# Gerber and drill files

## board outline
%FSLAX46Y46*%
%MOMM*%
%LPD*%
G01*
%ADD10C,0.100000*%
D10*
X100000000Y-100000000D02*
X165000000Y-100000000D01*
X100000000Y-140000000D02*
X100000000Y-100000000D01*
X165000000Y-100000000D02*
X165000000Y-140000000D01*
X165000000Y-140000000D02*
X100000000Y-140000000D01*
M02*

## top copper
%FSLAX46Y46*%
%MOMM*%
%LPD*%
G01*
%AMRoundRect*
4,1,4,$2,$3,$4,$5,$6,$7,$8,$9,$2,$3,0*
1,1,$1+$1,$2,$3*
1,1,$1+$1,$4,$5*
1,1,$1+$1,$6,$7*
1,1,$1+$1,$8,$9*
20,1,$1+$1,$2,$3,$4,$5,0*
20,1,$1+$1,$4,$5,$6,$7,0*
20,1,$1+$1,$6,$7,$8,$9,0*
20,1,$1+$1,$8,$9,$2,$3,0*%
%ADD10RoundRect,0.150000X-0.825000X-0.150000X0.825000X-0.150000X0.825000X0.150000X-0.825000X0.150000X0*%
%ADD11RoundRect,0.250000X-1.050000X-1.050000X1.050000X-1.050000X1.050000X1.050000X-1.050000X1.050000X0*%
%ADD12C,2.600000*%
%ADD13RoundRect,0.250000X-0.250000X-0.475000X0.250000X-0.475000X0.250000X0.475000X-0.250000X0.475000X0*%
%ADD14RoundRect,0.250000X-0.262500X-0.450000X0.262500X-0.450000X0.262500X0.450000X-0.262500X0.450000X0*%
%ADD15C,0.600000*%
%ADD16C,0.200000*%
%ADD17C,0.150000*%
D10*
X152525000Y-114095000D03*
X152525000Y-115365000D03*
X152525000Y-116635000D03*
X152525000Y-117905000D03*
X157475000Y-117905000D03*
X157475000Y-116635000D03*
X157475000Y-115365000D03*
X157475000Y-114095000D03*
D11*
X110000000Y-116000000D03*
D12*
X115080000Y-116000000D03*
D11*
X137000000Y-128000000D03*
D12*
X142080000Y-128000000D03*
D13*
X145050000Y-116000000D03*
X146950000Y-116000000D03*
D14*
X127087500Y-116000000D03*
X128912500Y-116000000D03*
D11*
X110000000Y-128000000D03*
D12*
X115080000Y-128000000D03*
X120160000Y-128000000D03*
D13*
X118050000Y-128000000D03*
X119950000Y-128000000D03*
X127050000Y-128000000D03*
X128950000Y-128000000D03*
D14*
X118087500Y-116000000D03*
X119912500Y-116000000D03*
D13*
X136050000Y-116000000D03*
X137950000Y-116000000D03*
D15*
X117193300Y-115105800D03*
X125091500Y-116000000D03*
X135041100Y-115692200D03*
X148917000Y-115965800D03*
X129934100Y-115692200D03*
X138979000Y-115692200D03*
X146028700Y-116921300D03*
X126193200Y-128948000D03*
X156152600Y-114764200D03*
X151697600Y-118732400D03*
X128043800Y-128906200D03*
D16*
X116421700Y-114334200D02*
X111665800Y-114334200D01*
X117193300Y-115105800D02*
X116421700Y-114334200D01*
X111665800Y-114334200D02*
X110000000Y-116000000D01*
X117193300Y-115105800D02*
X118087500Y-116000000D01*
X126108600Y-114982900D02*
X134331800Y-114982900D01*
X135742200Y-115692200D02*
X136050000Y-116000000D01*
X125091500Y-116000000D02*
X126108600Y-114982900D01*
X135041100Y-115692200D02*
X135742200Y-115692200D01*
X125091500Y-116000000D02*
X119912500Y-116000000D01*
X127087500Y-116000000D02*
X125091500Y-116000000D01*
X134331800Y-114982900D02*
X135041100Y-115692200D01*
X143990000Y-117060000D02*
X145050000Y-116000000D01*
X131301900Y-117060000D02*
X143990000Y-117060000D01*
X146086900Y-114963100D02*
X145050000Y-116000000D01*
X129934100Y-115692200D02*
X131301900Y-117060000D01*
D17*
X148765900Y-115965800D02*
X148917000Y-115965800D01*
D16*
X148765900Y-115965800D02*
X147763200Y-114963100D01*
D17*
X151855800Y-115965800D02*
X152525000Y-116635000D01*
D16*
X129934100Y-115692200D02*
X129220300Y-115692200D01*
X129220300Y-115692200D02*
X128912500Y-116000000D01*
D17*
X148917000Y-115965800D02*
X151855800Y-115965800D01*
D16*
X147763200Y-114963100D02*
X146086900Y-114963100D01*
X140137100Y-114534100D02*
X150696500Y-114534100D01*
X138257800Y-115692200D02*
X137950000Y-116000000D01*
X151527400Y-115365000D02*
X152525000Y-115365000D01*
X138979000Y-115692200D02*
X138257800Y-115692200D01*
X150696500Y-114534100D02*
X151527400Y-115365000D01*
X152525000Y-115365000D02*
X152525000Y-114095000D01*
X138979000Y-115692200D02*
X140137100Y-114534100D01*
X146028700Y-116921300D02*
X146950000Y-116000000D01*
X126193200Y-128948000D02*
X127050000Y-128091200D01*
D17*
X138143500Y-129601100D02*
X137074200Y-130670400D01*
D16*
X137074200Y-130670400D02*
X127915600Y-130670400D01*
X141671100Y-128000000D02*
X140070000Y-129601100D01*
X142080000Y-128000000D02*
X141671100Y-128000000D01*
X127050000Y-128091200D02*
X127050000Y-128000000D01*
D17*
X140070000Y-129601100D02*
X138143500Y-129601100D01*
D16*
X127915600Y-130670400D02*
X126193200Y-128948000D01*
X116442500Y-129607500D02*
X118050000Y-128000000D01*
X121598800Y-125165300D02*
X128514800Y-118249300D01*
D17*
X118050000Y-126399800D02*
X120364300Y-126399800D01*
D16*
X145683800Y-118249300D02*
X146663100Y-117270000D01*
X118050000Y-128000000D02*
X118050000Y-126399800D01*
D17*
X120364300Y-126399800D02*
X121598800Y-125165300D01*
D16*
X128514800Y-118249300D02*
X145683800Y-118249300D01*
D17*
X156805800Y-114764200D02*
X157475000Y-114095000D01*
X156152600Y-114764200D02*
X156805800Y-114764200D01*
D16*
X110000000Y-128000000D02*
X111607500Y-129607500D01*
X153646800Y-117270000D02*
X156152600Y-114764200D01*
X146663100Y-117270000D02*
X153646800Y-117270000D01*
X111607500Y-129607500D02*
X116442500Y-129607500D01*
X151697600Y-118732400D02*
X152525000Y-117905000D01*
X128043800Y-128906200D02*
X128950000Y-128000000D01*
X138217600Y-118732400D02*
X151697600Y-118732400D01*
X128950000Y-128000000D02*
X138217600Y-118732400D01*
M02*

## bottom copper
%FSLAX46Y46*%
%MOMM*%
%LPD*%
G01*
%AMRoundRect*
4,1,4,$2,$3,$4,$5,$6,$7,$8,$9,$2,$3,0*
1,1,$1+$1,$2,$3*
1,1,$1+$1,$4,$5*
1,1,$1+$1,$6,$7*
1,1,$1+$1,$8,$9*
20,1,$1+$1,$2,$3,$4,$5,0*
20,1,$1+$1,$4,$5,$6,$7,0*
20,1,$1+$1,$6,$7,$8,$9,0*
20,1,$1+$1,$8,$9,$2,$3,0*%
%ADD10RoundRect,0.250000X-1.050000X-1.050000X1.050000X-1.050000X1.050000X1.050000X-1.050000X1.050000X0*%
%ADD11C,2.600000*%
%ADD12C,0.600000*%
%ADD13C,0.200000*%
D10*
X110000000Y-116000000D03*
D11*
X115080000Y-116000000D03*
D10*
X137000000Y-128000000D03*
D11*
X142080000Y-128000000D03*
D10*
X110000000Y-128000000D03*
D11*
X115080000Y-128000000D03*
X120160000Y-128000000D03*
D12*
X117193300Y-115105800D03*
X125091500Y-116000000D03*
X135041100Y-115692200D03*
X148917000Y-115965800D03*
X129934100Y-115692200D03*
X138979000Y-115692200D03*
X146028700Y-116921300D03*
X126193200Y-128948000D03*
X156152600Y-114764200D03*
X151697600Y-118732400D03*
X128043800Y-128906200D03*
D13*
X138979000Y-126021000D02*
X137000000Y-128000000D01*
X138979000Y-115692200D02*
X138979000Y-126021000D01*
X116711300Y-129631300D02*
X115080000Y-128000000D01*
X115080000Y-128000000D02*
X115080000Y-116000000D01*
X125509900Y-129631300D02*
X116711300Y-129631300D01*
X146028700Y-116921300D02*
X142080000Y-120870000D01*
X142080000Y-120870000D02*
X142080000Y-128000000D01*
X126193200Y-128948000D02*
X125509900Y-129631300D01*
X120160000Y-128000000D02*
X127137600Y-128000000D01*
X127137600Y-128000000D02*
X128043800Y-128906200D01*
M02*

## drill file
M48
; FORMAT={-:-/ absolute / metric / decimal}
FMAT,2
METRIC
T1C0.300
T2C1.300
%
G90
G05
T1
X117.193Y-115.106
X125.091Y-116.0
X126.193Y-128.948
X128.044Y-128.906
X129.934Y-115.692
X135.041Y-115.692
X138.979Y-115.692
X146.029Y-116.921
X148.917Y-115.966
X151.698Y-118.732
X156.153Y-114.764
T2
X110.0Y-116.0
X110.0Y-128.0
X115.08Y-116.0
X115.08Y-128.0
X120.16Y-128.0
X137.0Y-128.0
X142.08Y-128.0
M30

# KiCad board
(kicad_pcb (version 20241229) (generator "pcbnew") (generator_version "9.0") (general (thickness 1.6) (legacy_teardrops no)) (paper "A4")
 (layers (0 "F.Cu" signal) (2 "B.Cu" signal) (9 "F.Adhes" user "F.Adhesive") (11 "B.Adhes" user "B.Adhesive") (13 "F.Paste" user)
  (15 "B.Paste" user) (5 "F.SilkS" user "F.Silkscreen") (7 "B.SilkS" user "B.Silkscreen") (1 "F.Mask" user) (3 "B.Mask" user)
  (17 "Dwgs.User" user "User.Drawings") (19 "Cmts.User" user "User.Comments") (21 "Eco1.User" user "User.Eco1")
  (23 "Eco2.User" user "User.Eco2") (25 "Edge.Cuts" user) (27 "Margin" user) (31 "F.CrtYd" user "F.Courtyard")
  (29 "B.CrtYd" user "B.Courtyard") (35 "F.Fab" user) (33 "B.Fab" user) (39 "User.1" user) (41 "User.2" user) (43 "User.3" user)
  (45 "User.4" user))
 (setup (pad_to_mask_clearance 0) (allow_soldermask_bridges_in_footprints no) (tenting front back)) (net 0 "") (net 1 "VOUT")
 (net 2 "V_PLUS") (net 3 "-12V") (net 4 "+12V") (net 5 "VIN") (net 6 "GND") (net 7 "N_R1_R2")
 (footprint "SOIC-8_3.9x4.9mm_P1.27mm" (layer "F.Cu") (at 155 116)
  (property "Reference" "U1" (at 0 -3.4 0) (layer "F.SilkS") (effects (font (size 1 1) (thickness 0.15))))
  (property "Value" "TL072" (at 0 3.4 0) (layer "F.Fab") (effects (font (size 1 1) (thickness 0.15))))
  (pad "1" smd roundrect (at -2.475 -1.905) (size 1.95 0.6) (layers "F.Cu" "F.Mask" "F.Paste") (roundrect_rratio 0.25) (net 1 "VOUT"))
  (pad "2" smd roundrect (at -2.475 -0.635) (size 1.95 0.6) (layers "F.Cu" "F.Mask" "F.Paste") (roundrect_rratio 0.25) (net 1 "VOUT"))
  (pad "3" smd roundrect (at -2.475 0.635) (size 1.95 0.6) (layers "F.Cu" "F.Mask" "F.Paste") (roundrect_rratio 0.25) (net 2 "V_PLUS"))
  (pad "4" smd roundrect (at -2.475 1.905) (size 1.95 0.6) (layers "F.Cu" "F.Mask" "F.Paste") (roundrect_rratio 0.25) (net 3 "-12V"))
  (pad "5" smd roundrect (at 2.475 1.905) (size 1.95 0.6) (layers "F.Cu" "F.Mask" "F.Paste") (roundrect_rratio 0.25))
  (pad "6" smd roundrect (at 2.475 0.635) (size 1.95 0.6) (layers "F.Cu" "F.Mask" "F.Paste") (roundrect_rratio 0.25))
  (pad "7" smd roundrect (at 2.475 -0.635) (size 1.95 0.6) (layers "F.Cu" "F.Mask" "F.Paste") (roundrect_rratio 0.25))
  (pad "8" smd roundrect (at 2.475 -1.905) (size 1.95 0.6) (layers "F.Cu" "F.Mask" "F.Paste") (roundrect_rratio 0.25) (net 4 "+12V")))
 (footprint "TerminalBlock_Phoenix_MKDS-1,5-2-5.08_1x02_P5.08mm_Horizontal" (layer "F.Cu") (at 110 116)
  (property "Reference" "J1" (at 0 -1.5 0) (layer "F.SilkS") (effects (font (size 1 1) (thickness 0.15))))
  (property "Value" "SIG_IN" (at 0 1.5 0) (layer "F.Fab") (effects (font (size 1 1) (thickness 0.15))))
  (pad "1" thru_hole roundrect (at 0 0) (size 2.6 2.6) (drill 1.3) (layers "*.Cu" "*.Mask") (remove_unused_layers no)
   (roundrect_rratio 0.096154) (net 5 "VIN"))
  (pad "2" thru_hole circle (at 5.08 0) (size 2.6 2.6) (drill 1.3) (layers "*.Cu" "*.Mask") (remove_unused_layers no) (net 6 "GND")))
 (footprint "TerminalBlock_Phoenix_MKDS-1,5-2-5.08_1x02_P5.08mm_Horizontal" (layer "F.Cu") (at 137 128)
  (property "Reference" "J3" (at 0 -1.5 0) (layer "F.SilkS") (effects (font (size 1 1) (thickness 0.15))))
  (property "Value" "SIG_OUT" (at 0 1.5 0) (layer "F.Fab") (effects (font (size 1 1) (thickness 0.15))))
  (pad "1" thru_hole roundrect (at 0 0) (size 2.6 2.6) (drill 1.3) (layers "*.Cu" "*.Mask") (remove_unused_layers no)
   (roundrect_rratio 0.096154) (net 1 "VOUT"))
  (pad "2" thru_hole circle (at 5.08 0) (size 2.6 2.6) (drill 1.3) (layers "*.Cu" "*.Mask") (remove_unused_layers no) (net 6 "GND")))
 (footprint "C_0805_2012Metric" (layer "F.Cu") (at 146 116)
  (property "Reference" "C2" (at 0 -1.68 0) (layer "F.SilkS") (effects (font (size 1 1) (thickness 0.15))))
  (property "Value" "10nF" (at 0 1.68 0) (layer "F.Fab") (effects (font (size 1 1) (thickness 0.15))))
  (pad "1" smd roundrect (at -0.95 0) (size 1 1.45) (layers "F.Cu" "F.Mask" "F.Paste") (roundrect_rratio 0.25) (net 2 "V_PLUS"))
  (pad "2" smd roundrect (at 0.95 0) (size 1 1.45) (layers "F.Cu" "F.Mask" "F.Paste") (roundrect_rratio 0.25) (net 6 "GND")))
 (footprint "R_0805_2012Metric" (layer "F.Cu") (at 128 116)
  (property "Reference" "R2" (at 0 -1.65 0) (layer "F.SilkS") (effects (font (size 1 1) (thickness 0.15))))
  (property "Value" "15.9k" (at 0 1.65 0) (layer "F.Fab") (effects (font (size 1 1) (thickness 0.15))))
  (pad "1" smd roundrect (at -0.9125 0) (size 1.025 1.4) (layers "F.Cu" "F.Mask" "F.Paste") (roundrect_rratio 0.243902) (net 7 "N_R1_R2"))
  (pad "2" smd roundrect (at 0.9125 0) (size 1.025 1.4) (layers "F.Cu" "F.Mask" "F.Paste") (roundrect_rratio 0.243902) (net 2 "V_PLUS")))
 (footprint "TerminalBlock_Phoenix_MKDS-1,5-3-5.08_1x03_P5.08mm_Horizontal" (layer "F.Cu") (at 110 128)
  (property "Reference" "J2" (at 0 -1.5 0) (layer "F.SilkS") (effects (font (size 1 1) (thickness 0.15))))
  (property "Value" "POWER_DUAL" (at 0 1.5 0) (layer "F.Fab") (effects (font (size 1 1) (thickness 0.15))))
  (pad "1" thru_hole roundrect (at 0 0) (size 2.6 2.6) (drill 1.3) (layers "*.Cu" "*.Mask") (remove_unused_layers no)
   (roundrect_rratio 0.096154) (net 4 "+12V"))
  (pad "2" thru_hole circle (at 5.08 0) (size 2.6 2.6) (drill 1.3) (layers "*.Cu" "*.Mask") (remove_unused_layers no) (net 6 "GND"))
  (pad "3" thru_hole circle (at 10.16 0) (size 2.6 2.6) (drill 1.3) (layers "*.Cu" "*.Mask") (remove_unused_layers no) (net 3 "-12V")))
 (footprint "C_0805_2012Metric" (layer "F.Cu") (at 119 128)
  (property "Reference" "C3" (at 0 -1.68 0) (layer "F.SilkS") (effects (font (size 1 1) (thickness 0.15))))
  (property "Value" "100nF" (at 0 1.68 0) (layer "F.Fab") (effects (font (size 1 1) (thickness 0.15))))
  (pad "1" smd roundrect (at -0.95 0) (size 1 1.45) (layers "F.Cu" "F.Mask" "F.Paste") (roundrect_rratio 0.25) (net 4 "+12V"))
  (pad "2" smd roundrect (at 0.95 0) (size 1 1.45) (layers "F.Cu" "F.Mask" "F.Paste") (roundrect_rratio 0.25) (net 6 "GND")))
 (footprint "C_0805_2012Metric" (layer "F.Cu") (at 128 128)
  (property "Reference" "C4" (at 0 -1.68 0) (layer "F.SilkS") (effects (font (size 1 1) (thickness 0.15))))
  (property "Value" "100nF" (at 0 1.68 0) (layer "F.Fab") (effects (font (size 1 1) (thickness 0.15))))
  (pad "1" smd roundrect (at -0.95 0) (size 1 1.45) (layers "F.Cu" "F.Mask" "F.Paste") (roundrect_rratio 0.25) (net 6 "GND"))
  (pad "2" smd roundrect (at 0.95 0) (size 1 1.45) (layers "F.Cu" "F.Mask" "F.Paste") (roundrect_rratio 0.25) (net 3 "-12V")))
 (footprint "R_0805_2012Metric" (layer "F.Cu") (at 119 116)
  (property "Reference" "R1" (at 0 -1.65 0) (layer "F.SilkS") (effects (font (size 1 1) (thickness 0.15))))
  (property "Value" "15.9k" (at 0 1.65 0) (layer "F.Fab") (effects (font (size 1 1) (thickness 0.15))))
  (pad "1" smd roundrect (at -0.9125 0) (size 1.025 1.4) (layers "F.Cu" "F.Mask" "F.Paste") (roundrect_rratio 0.243902) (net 5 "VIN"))
  (pad "2" smd roundrect (at 0.9125 0) (size 1.025 1.4) (layers "F.Cu" "F.Mask" "F.Paste") (roundrect_rratio 0.243902) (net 7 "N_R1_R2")))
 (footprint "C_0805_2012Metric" (layer "F.Cu") (at 137 116)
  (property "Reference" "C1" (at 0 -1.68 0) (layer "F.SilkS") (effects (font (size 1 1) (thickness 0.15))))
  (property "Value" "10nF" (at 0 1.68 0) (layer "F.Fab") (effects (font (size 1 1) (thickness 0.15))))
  (pad "1" smd roundrect (at -0.95 0) (size 1 1.45) (layers "F.Cu" "F.Mask" "F.Paste") (roundrect_rratio 0.25) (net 7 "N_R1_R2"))
  (pad "2" smd roundrect (at 0.95 0) (size 1 1.45) (layers "F.Cu" "F.Mask" "F.Paste") (roundrect_rratio 0.25) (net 1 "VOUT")))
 (gr_line (start 100 100) (end 165 100) (stroke (width 0.1) (type default)) (layer "Edge.Cuts"))
 (gr_line (start 100 140) (end 100 100) (stroke (width 0.1) (type default)) (layer "Edge.Cuts"))
 (gr_line (start 165 100) (end 165 140) (stroke (width 0.1) (type default)) (layer "Edge.Cuts"))
 (gr_line (start 165 140) (end 100 140) (stroke (width 0.1) (type default)) (layer "Edge.Cuts"))
 (segment (start 116.4217 114.3342) (end 111.6658 114.3342) (width 0.2) (layer "F.Cu") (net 5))
 (segment (start 117.1933 115.1058) (end 116.4217 114.3342) (width 0.2) (layer "F.Cu") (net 5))
 (segment (start 111.6658 114.3342) (end 110 116) (width 0.2) (layer "F.Cu") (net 5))
 (segment (start 117.1933 115.1058) (end 118.0875 116) (width 0.2) (layer "F.Cu") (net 5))
 (via (at 117.1933 115.1058) (size 0.6) (drill 0.3) (layers "F.Cu" "B.Cu") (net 5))
 (segment (start 126.1086 114.9829) (end 134.3318 114.9829) (width 0.2) (layer "F.Cu") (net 7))
 (segment (start 135.7422 115.6922) (end 136.05 116) (width 0.2) (layer "F.Cu") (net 7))
 (segment (start 125.0915 116) (end 126.1086 114.9829) (width 0.2) (layer "F.Cu") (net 7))
 (segment (start 135.0411 115.6922) (end 135.7422 115.6922) (width 0.2) (layer "F.Cu") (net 7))
 (segment (start 125.0915 116) (end 119.9125 116) (width 0.2) (layer "F.Cu") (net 7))
 (segment (start 127.0875 116) (end 125.0915 116) (width 0.2) (layer "F.Cu") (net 7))
 (segment (start 134.3318 114.9829) (end 135.0411 115.6922) (width 0.2) (layer "F.Cu") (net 7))
 (via (at 125.0915 116) (size 0.6) (drill 0.3) (layers "F.Cu" "B.Cu") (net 7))
 (via (at 135.0411 115.6922) (size 0.6) (drill 0.3) (layers "F.Cu" "B.Cu") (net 7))
 (segment (start 143.99 117.06) (end 145.05 116) (width 0.2) (layer "F.Cu") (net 2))
 (segment (start 131.3019 117.06) (end 143.99 117.06) (width 0.2) (layer "F.Cu") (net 2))
 (segment (start 146.0869 114.9631) (end 145.05 116) (width 0.2) (layer "F.Cu") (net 2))
 (segment (start 129.9341 115.6922) (end 131.3019 117.06) (width 0.2) (layer "F.Cu") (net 2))
 (segment (start 148.7659 115.9658) (end 148.917 115.9658) (width 0.15) (layer "F.Cu") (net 2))
 (segment (start 148.7659 115.9658) (end 147.7632 114.9631) (width 0.2) (layer "F.Cu") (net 2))
 (segment (start 151.8558 115.9658) (end 152.525 116.635) (width 0.15) (layer "F.Cu") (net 2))
 (segment (start 129.9341 115.6922) (end 129.2203 115.6922) (width 0.2) (layer "F.Cu") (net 2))
 (segment (start 129.2203 115.6922) (end 128.9125 116) (width 0.2) (layer "F.Cu") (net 2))
 (segment (start 148.917 115.9658) (end 151.8558 115.9658) (width 0.15) (layer "F.Cu") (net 2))
 (segment (start 147.7632 114.9631) (end 146.0869 114.9631) (width 0.2) (layer "F.Cu") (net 2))
 (via (at 148.917 115.9658) (size 0.6) (drill 0.3) (layers "F.Cu" "B.Cu") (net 2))
 (via (at 129.9341 115.6922) (size 0.6) (drill 0.3) (layers "F.Cu" "B.Cu") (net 2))
 (segment (start 140.1371 114.5341) (end 150.6965 114.5341) (width 0.2) (layer "F.Cu") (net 1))
 (segment (start 138.2578 115.6922) (end 137.95 116) (width 0.2) (layer "F.Cu") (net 1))
 (segment (start 151.5274 115.365) (end 152.525 115.365) (width 0.2) (layer "F.Cu") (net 1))
 (segment (start 138.979 115.6922) (end 138.2578 115.6922) (width 0.2) (layer "F.Cu") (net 1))
 (segment (start 150.6965 114.5341) (end 151.5274 115.365) (width 0.2) (layer "F.Cu") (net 1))
 (segment (start 152.525 115.365) (end 152.525 114.095) (width 0.2) (layer "F.Cu") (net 1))
 (segment (start 138.979 115.6922) (end 140.1371 114.5341) (width 0.2) (layer "F.Cu") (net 1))
 (via (at 138.979 115.6922) (size 0.6) (drill 0.3) (layers "F.Cu" "B.Cu") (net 1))
 (segment (start 138.979 126.021) (end 137 128) (width 0.2) (layer "B.Cu") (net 1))
 (segment (start 138.979 115.6922) (end 138.979 126.021) (width 0.2) (layer "B.Cu") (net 1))
 (segment (start 146.0287 116.9213) (end 146.95 116) (width 0.2) (layer "F.Cu") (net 6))
 (segment (start 126.1932 128.948) (end 127.05 128.0912) (width 0.2) (layer "F.Cu") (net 6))
 (segment (start 138.1435 129.6011) (end 137.0742 130.6704) (width 0.15) (layer "F.Cu") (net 6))
 (segment (start 137.0742 130.6704) (end 127.9156 130.6704) (width 0.2) (layer "F.Cu") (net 6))
 (segment (start 141.6711 128) (end 140.07 129.6011) (width 0.2) (layer "F.Cu") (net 6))
 (segment (start 142.08 128) (end 141.6711 128) (width 0.2) (layer "F.Cu") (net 6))
 (segment (start 127.05 128.0912) (end 127.05 128) (width 0.2) (layer "F.Cu") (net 6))
 (segment (start 140.07 129.6011) (end 138.1435 129.6011) (width 0.15) (layer "F.Cu") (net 6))
 (segment (start 127.9156 130.6704) (end 126.1932 128.948) (width 0.2) (layer "F.Cu") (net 6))
 (via (at 146.0287 116.9213) (size 0.6) (drill 0.3) (layers "F.Cu" "B.Cu") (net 6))
 (via (at 126.1932 128.948) (size 0.6) (drill 0.3) (layers "F.Cu" "B.Cu") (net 6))
 (segment (start 116.7113 129.6313) (end 115.08 128) (width 0.2) (layer "B.Cu") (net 6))
 (segment (start 115.08 128) (end 115.08 116) (width 0.2) (layer "B.Cu") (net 6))
 (segment (start 125.5099 129.6313) (end 116.7113 129.6313) (width 0.2) (layer "B.Cu") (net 6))
 (segment (start 146.0287 116.9213) (end 142.08 120.87) (width 0.2) (layer "B.Cu") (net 6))
 (segment (start 142.08 120.87) (end 142.08 128) (width 0.2) (layer "B.Cu") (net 6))
 (segment (start 126.1932 128.948) (end 125.5099 129.6313) (width 0.2) (layer "B.Cu") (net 6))
 (segment (start 116.4425 129.6075) (end 118.05 128) (width 0.2) (layer "F.Cu") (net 4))
 (segment (start 121.5988 125.1653) (end 128.5148 118.2493) (width 0.2) (layer "F.Cu") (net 4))
 (segment (start 118.05 126.3998) (end 120.3643 126.3998) (width 0.15) (layer "F.Cu") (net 4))
 (segment (start 145.6838 118.2493) (end 146.6631 117.27) (width 0.2) (layer "F.Cu") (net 4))
 (segment (start 118.05 128) (end 118.05 126.3998) (width 0.2) (layer "F.Cu") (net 4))
 (segment (start 120.3643 126.3998) (end 121.5988 125.1653) (width 0.15) (layer "F.Cu") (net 4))
 (segment (start 128.5148 118.2493) (end 145.6838 118.2493) (width 0.2) (layer "F.Cu") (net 4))
 (segment (start 156.8058 114.7642) (end 157.475 114.095) (width 0.15) (layer "F.Cu") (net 4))
 (segment (start 156.1526 114.7642) (end 156.8058 114.7642) (width 0.15) (layer "F.Cu") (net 4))
 (segment (start 110 128) (end 111.6075 129.6075) (width 0.2) (layer "F.Cu") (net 4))
 (segment (start 153.6468 117.27) (end 156.1526 114.7642) (width 0.2) (layer "F.Cu") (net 4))
 (segment (start 146.6631 117.27) (end 153.6468 117.27) (width 0.2) (layer "F.Cu") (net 4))
 (segment (start 111.6075 129.6075) (end 116.4425 129.6075) (width 0.2) (layer "F.Cu") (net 4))
 (via (at 156.1526 114.7642) (size 0.6) (drill 0.3) (layers "F.Cu" "B.Cu") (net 4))
 (segment (start 151.6976 118.7324) (end 152.525 117.905) (width 0.2) (layer "F.Cu") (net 3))
 (segment (start 128.0438 128.9062) (end 128.95 128) (width 0.2) (layer "F.Cu") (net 3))
 (segment (start 138.2176 118.7324) (end 151.6976 118.7324) (width 0.2) (layer "F.Cu") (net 3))
 (segment (start 128.95 128) (end 138.2176 118.7324) (width 0.2) (layer "F.Cu") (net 3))
 (via (at 151.6976 118.7324) (size 0.6) (drill 0.3) (layers "F.Cu" "B.Cu") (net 3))
 (via (at 128.0438 128.9062) (size 0.6) (drill 0.3) (layers "F.Cu" "B.Cu") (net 3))
 (segment (start 120.16 128) (end 127.1376 128) (width 0.2) (layer "B.Cu") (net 3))
 (segment (start 127.1376 128) (end 128.0438 128.9062) (width 0.2) (layer "B.Cu") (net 3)))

